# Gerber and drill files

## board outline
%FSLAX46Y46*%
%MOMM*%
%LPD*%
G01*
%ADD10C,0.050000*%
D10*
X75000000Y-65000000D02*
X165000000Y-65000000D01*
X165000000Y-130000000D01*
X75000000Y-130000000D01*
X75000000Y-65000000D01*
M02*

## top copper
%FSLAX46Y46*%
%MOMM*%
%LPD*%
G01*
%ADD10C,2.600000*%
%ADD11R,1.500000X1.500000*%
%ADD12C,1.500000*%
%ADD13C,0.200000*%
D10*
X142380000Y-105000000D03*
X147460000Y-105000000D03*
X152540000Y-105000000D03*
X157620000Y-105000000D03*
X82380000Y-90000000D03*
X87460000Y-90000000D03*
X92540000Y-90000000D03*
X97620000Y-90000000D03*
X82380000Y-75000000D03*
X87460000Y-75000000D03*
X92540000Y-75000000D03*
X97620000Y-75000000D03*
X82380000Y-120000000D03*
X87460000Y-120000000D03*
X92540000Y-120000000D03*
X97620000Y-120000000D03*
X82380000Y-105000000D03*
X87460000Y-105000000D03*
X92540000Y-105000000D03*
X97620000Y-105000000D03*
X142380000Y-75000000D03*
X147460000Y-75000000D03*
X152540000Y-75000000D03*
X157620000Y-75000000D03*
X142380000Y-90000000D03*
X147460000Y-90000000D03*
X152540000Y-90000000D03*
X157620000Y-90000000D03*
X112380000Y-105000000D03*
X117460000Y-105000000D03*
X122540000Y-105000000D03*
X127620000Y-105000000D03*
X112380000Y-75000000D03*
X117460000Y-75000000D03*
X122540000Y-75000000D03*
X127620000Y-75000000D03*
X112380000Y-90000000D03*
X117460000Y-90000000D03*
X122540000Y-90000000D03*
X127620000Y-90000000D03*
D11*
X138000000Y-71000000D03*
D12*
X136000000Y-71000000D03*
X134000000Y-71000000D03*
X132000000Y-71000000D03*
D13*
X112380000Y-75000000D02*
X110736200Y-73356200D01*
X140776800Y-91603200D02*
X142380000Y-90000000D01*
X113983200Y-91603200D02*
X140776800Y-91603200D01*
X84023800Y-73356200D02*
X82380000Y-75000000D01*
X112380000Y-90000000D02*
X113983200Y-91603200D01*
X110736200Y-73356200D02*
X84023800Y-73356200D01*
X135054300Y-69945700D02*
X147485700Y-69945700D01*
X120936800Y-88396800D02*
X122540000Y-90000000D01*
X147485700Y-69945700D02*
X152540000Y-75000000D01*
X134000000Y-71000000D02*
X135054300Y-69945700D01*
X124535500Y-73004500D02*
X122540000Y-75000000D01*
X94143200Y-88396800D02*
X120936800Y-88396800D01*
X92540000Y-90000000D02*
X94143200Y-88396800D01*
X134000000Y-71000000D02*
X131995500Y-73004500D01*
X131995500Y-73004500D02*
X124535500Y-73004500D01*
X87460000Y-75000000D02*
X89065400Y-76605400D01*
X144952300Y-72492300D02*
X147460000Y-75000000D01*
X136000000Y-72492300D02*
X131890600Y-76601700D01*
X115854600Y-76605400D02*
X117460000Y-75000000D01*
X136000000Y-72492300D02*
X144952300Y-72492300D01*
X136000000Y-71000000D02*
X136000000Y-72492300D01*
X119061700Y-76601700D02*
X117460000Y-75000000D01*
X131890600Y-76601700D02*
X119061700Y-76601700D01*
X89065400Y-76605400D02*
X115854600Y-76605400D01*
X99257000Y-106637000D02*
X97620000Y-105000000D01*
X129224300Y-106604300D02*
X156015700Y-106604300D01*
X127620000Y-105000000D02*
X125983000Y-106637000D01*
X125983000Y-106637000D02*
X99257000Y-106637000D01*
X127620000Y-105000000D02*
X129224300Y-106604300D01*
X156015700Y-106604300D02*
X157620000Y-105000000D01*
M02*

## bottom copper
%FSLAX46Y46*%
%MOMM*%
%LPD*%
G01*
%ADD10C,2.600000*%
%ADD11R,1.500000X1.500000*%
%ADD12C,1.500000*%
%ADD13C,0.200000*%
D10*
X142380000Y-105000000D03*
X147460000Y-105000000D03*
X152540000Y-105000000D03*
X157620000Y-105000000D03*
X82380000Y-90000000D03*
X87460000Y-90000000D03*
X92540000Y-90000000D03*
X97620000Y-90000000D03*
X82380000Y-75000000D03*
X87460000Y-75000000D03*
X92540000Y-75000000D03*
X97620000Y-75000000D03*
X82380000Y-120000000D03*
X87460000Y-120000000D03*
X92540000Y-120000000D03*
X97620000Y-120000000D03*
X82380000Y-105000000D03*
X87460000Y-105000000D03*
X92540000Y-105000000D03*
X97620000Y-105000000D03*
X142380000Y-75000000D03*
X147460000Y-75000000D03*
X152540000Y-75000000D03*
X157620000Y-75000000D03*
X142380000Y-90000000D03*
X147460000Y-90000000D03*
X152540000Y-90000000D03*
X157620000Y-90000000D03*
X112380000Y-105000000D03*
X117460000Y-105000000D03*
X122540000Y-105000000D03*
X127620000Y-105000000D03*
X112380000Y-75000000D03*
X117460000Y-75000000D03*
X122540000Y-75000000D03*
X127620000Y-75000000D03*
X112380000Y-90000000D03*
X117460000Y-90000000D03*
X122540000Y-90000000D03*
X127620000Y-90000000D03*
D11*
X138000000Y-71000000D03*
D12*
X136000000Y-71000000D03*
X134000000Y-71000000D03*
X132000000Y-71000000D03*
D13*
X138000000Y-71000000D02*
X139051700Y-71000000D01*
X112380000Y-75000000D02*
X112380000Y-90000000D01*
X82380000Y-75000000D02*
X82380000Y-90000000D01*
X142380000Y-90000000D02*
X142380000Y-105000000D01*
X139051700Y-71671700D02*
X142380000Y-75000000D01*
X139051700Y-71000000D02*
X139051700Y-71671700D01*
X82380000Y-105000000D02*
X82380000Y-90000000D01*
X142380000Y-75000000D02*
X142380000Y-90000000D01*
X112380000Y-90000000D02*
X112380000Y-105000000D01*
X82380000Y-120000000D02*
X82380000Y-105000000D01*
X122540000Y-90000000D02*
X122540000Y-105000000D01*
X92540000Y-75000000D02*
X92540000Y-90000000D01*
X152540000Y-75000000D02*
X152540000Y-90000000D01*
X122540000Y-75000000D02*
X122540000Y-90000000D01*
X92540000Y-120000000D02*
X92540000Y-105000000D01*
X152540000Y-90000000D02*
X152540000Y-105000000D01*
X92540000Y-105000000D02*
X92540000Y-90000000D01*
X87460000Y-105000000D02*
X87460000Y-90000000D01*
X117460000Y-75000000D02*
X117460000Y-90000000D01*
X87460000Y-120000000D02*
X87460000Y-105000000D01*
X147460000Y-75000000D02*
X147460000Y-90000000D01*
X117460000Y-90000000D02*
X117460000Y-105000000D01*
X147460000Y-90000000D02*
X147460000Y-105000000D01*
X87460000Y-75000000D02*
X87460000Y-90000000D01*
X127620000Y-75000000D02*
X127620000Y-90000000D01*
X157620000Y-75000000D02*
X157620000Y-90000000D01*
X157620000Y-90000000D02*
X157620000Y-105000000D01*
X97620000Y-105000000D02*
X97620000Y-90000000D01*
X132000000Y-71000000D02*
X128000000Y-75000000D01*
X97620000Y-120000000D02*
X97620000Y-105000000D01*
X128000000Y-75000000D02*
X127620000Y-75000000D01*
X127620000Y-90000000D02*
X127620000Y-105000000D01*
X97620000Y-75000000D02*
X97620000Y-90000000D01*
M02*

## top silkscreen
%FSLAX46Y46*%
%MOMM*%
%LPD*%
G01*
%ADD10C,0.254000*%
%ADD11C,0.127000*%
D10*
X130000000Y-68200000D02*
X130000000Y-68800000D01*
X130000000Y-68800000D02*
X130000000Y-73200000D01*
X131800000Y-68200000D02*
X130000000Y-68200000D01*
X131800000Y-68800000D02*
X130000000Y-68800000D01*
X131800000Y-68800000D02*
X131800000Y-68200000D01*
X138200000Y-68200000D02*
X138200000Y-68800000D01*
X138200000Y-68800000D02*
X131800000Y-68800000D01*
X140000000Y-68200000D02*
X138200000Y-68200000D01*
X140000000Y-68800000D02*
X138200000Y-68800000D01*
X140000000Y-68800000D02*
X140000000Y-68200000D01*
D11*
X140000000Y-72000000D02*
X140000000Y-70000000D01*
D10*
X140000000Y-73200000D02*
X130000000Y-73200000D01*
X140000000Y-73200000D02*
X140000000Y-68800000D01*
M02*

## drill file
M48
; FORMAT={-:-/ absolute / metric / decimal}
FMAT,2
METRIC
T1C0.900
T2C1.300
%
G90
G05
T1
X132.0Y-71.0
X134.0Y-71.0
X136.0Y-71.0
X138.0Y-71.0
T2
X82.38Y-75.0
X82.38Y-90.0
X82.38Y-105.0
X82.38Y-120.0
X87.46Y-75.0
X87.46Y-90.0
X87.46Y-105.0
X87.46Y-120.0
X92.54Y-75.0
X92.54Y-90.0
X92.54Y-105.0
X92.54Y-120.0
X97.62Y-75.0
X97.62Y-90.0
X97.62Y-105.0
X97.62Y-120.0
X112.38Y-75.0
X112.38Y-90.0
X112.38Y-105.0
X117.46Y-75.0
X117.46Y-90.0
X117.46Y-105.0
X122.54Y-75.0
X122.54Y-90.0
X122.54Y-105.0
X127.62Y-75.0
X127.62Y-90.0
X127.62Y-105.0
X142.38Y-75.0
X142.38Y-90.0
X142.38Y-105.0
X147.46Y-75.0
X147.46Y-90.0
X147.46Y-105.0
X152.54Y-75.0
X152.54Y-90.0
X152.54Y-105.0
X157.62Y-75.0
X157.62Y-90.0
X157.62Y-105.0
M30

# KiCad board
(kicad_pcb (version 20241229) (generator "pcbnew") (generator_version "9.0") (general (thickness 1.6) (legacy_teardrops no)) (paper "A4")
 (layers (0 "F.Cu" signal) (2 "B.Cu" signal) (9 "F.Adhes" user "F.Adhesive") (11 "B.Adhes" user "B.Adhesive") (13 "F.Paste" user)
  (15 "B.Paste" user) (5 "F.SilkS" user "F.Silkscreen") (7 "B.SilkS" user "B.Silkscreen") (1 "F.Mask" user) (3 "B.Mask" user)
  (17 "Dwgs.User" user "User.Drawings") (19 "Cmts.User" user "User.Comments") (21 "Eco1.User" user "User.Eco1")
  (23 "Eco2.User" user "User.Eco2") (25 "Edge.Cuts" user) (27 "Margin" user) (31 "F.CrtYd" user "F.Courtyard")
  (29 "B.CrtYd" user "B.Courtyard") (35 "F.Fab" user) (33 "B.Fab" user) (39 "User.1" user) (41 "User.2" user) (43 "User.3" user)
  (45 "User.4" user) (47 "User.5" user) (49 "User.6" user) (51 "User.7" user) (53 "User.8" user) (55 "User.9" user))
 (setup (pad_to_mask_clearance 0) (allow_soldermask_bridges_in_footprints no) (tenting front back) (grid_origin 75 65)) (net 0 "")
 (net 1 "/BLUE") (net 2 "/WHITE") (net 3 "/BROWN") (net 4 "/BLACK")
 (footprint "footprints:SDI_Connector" (layer "F.Cu") (at 150 105)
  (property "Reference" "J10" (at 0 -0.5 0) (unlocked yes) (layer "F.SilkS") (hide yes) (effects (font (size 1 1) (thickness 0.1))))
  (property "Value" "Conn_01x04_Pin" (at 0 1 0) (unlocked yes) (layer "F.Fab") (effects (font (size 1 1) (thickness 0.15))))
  (pad "1" thru_hole circle (at -7.62 0) (size 2.6 2.6) (drill 1.3) (layers "*.Cu" "*.Mask") (remove_unused_layers no) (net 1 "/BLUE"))
  (pad "2" thru_hole circle (at -2.54 0) (size 2.6 2.6) (drill 1.3) (layers "*.Cu" "*.Mask") (remove_unused_layers no) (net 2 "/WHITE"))
  (pad "3" thru_hole circle (at 2.54 0) (size 2.6 2.6) (drill 1.3) (layers "*.Cu" "*.Mask") (remove_unused_layers no) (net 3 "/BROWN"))
  (pad "4" thru_hole circle (at 7.62 0) (size 2.6 2.6) (drill 1.3) (layers "*.Cu" "*.Mask") (remove_unused_layers no) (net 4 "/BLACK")))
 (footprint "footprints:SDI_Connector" (layer "F.Cu") (at 90 90)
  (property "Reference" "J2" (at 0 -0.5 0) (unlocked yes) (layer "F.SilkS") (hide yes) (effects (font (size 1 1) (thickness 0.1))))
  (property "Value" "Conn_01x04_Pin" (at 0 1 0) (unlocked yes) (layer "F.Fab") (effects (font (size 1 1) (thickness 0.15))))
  (pad "1" thru_hole circle (at -7.62 0) (size 2.6 2.6) (drill 1.3) (layers "*.Cu" "*.Mask") (remove_unused_layers no) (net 1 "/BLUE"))
  (pad "2" thru_hole circle (at -2.54 0) (size 2.6 2.6) (drill 1.3) (layers "*.Cu" "*.Mask") (remove_unused_layers no) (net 2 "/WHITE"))
  (pad "3" thru_hole circle (at 2.54 0) (size 2.6 2.6) (drill 1.3) (layers "*.Cu" "*.Mask") (remove_unused_layers no) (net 3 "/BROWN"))
  (pad "4" thru_hole circle (at 7.62 0) (size 2.6 2.6) (drill 1.3) (layers "*.Cu" "*.Mask") (remove_unused_layers no) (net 4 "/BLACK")))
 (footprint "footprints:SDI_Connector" (layer "F.Cu") (at 90 75)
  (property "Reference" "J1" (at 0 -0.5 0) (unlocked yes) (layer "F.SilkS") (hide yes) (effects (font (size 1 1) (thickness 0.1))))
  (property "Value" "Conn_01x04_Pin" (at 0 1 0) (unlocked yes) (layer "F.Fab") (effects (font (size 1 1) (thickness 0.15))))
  (pad "1" thru_hole circle (at -7.62 0) (size 2.6 2.6) (drill 1.3) (layers "*.Cu" "*.Mask") (remove_unused_layers no) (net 1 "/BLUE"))
  (pad "2" thru_hole circle (at -2.54 0) (size 2.6 2.6) (drill 1.3) (layers "*.Cu" "*.Mask") (remove_unused_layers no) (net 2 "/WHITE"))
  (pad "3" thru_hole circle (at 2.54 0) (size 2.6 2.6) (drill 1.3) (layers "*.Cu" "*.Mask") (remove_unused_layers no) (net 3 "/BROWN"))
  (pad "4" thru_hole circle (at 7.62 0) (size 2.6 2.6) (drill 1.3) (layers "*.Cu" "*.Mask") (remove_unused_layers no) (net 4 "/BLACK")))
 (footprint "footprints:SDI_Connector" (layer "F.Cu") (at 90 120)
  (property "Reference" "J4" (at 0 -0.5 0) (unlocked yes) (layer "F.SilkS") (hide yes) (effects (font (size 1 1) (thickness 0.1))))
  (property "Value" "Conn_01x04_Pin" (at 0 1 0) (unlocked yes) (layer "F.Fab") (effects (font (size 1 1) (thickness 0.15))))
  (pad "1" thru_hole circle (at -7.62 0) (size 2.6 2.6) (drill 1.3) (layers "*.Cu" "*.Mask") (remove_unused_layers no) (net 1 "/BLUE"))
  (pad "2" thru_hole circle (at -2.54 0) (size 2.6 2.6) (drill 1.3) (layers "*.Cu" "*.Mask") (remove_unused_layers no) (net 2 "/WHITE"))
  (pad "3" thru_hole circle (at 2.54 0) (size 2.6 2.6) (drill 1.3) (layers "*.Cu" "*.Mask") (remove_unused_layers no) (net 3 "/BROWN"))
  (pad "4" thru_hole circle (at 7.62 0) (size 2.6 2.6) (drill 1.3) (layers "*.Cu" "*.Mask") (remove_unused_layers no) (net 4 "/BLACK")))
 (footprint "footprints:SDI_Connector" (layer "F.Cu") (at 90 105)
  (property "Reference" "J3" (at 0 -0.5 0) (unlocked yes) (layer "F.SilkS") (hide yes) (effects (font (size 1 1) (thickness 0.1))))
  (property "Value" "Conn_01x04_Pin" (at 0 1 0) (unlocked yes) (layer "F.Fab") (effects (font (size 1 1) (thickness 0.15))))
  (pad "1" thru_hole circle (at -7.62 0) (size 2.6 2.6) (drill 1.3) (layers "*.Cu" "*.Mask") (remove_unused_layers no) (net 1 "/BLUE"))
  (pad "2" thru_hole circle (at -2.54 0) (size 2.6 2.6) (drill 1.3) (layers "*.Cu" "*.Mask") (remove_unused_layers no) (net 2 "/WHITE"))
  (pad "3" thru_hole circle (at 2.54 0) (size 2.6 2.6) (drill 1.3) (layers "*.Cu" "*.Mask") (remove_unused_layers no) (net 3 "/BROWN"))
  (pad "4" thru_hole circle (at 7.62 0) (size 2.6 2.6) (drill 1.3) (layers "*.Cu" "*.Mask") (remove_unused_layers no) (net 4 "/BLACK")))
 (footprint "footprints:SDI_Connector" (layer "F.Cu") (at 150 75)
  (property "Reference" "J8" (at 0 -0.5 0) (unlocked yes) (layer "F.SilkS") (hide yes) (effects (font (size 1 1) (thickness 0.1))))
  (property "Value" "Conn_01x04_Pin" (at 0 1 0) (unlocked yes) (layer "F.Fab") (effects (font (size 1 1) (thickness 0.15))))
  (pad "1" thru_hole circle (at -7.62 0) (size 2.6 2.6) (drill 1.3) (layers "*.Cu" "*.Mask") (remove_unused_layers no) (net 1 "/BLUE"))
  (pad "2" thru_hole circle (at -2.54 0) (size 2.6 2.6) (drill 1.3) (layers "*.Cu" "*.Mask") (remove_unused_layers no) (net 2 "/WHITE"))
  (pad "3" thru_hole circle (at 2.54 0) (size 2.6 2.6) (drill 1.3) (layers "*.Cu" "*.Mask") (remove_unused_layers no) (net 3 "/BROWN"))
  (pad "4" thru_hole circle (at 7.62 0) (size 2.6 2.6) (drill 1.3) (layers "*.Cu" "*.Mask") (remove_unused_layers no) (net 4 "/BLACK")))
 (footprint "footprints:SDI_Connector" (layer "F.Cu") (at 150 90)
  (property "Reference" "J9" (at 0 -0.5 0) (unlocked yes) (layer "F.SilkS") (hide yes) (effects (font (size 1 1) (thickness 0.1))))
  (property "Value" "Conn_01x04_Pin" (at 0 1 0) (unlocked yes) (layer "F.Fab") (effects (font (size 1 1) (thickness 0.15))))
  (pad "1" thru_hole circle (at -7.62 0) (size 2.6 2.6) (drill 1.3) (layers "*.Cu" "*.Mask") (remove_unused_layers no) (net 1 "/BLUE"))
  (pad "2" thru_hole circle (at -2.54 0) (size 2.6 2.6) (drill 1.3) (layers "*.Cu" "*.Mask") (remove_unused_layers no) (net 2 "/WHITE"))
  (pad "3" thru_hole circle (at 2.54 0) (size 2.6 2.6) (drill 1.3) (layers "*.Cu" "*.Mask") (remove_unused_layers no) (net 3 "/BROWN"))
  (pad "4" thru_hole circle (at 7.62 0) (size 2.6 2.6) (drill 1.3) (layers "*.Cu" "*.Mask") (remove_unused_layers no) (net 4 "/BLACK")))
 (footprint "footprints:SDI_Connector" (layer "F.Cu") (at 120 105)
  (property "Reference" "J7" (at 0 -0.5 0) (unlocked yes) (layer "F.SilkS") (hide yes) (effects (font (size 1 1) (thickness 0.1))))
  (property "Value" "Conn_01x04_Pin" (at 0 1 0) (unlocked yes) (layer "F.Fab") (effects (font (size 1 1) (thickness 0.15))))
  (pad "1" thru_hole circle (at -7.62 0) (size 2.6 2.6) (drill 1.3) (layers "*.Cu" "*.Mask") (remove_unused_layers no) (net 1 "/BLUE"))
  (pad "2" thru_hole circle (at -2.54 0) (size 2.6 2.6) (drill 1.3) (layers "*.Cu" "*.Mask") (remove_unused_layers no) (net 2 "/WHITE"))
  (pad "3" thru_hole circle (at 2.54 0) (size 2.6 2.6) (drill 1.3) (layers "*.Cu" "*.Mask") (remove_unused_layers no) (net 3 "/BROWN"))
  (pad "4" thru_hole circle (at 7.62 0) (size 2.6 2.6) (drill 1.3) (layers "*.Cu" "*.Mask") (remove_unused_layers no) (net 4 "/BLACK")))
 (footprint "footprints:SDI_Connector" (layer "F.Cu") (at 120 75)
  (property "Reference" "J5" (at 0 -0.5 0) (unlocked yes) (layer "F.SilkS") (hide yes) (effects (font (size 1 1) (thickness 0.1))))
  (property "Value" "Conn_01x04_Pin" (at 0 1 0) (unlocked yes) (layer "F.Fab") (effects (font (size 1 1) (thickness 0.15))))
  (pad "1" thru_hole circle (at -7.62 0) (size 2.6 2.6) (drill 1.3) (layers "*.Cu" "*.Mask") (remove_unused_layers no) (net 1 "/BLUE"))
  (pad "2" thru_hole circle (at -2.54 0) (size 2.6 2.6) (drill 1.3) (layers "*.Cu" "*.Mask") (remove_unused_layers no) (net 2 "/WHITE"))
  (pad "3" thru_hole circle (at 2.54 0) (size 2.6 2.6) (drill 1.3) (layers "*.Cu" "*.Mask") (remove_unused_layers no) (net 3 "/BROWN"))
  (pad "4" thru_hole circle (at 7.62 0) (size 2.6 2.6) (drill 1.3) (layers "*.Cu" "*.Mask") (remove_unused_layers no) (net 4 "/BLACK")))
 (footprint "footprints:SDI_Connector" (layer "F.Cu") (at 120 90)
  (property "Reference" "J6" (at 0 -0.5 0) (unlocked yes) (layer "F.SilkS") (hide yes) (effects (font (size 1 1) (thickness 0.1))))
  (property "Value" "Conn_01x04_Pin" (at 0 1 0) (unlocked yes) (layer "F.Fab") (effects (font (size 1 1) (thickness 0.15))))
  (pad "1" thru_hole circle (at -7.62 0) (size 2.6 2.6) (drill 1.3) (layers "*.Cu" "*.Mask") (remove_unused_layers no) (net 1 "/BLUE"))
  (pad "2" thru_hole circle (at -2.54 0) (size 2.6 2.6) (drill 1.3) (layers "*.Cu" "*.Mask") (remove_unused_layers no) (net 2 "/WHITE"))
  (pad "3" thru_hole circle (at 2.54 0) (size 2.6 2.6) (drill 1.3) (layers "*.Cu" "*.Mask") (remove_unused_layers no) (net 3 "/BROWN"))
  (pad "4" thru_hole circle (at 7.62 0) (size 2.6 2.6) (drill 1.3) (layers "*.Cu" "*.Mask") (remove_unused_layers no) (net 4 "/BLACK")))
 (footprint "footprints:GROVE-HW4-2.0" (layer "F.Cu") (at 135 71 180)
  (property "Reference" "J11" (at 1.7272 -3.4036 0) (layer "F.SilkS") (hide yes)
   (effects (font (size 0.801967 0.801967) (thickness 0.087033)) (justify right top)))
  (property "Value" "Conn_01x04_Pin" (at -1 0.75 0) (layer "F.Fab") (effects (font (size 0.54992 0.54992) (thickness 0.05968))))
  (fp_line (start 5 2.8) (end 5 2.2) (stroke (width 0.254) (type solid)) (layer "F.SilkS"))
  (fp_line (start 5 2.2) (end 5 -2.2) (stroke (width 0.254) (type solid)) (layer "F.SilkS"))
  (fp_line (start 3.2 2.8) (end 5 2.8) (stroke (width 0.254) (type solid)) (layer "F.SilkS"))
  (fp_line (start 3.2 2.2) (end 5 2.2) (stroke (width 0.254) (type solid)) (layer "F.SilkS"))
  (fp_line (start 3.2 2.2) (end 3.2 2.8) (stroke (width 0.254) (type solid)) (layer "F.SilkS"))
  (fp_line (start -3.2 2.8) (end -3.2 2.2) (stroke (width 0.254) (type solid)) (layer "F.SilkS"))
  (fp_line (start -3.2 2.2) (end 3.2 2.2) (stroke (width 0.254) (type solid)) (layer "F.SilkS"))
  (fp_line (start -5 2.8) (end -3.2 2.8) (stroke (width 0.254) (type solid)) (layer "F.SilkS"))
  (fp_line (start -5 2.2) (end -3.2 2.2) (stroke (width 0.254) (type solid)) (layer "F.SilkS"))
  (fp_line (start -5 2.2) (end -5 2.8) (stroke (width 0.254) (type solid)) (layer "F.SilkS"))
  (fp_line (start -5 -1) (end -5 1) (stroke (width 0.127) (type solid)) (layer "F.SilkS"))
  (fp_line (start -5 -2.2) (end 5 -2.2) (stroke (width 0.254) (type solid)) (layer "F.SilkS"))
  (fp_line (start -5 -2.2) (end -5 2.2) (stroke (width 0.254) (type solid)) (layer "F.SilkS"))
  (pad "1" thru_hole rect (at -3 0 180) (size 1.5 1.5) (drill 0.9) (layers "*.Cu" "*.Mask") (remove_unused_layers no) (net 1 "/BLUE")
   (solder_mask_margin 0.1016) (thermal_bridge_angle 45))
  (pad "2" thru_hole circle (at -1 0 180) (size 1.5 1.5) (drill 0.9) (layers "*.Cu" "*.Mask") (remove_unused_layers no) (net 2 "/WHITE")
   (solder_mask_margin 0.1016))
  (pad "3" thru_hole circle (at 1 0 180) (size 1.5 1.5) (drill 0.9) (layers "*.Cu" "*.Mask") (remove_unused_layers no) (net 3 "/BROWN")
   (solder_mask_margin 0.1016))
  (pad "4" thru_hole circle (at 3 0 180) (size 1.5 1.5) (drill 0.9) (layers "*.Cu" "*.Mask") (remove_unused_layers no) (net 4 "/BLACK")
   (solder_mask_margin 0.1016)))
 (gr_rect (start 75 65) (end 165 130) (stroke (width 0.05) (type solid)) (fill no) (layer "Edge.Cuts"))
 (segment (start 112.38 75) (end 110.7362 73.3562) (width 0.2) (layer "F.Cu") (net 1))
 (segment (start 140.7768 91.6032) (end 142.38 90) (width 0.2) (layer "F.Cu") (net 1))
 (segment (start 113.9832 91.6032) (end 140.7768 91.6032) (width 0.2) (layer "F.Cu") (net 1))
 (segment (start 84.0238 73.3562) (end 82.38 75) (width 0.2) (layer "F.Cu") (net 1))
 (segment (start 112.38 90) (end 113.9832 91.6032) (width 0.2) (layer "F.Cu") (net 1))
 (segment (start 110.7362 73.3562) (end 84.0238 73.3562) (width 0.2) (layer "F.Cu") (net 1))
 (segment (start 138 71) (end 139.0517 71) (width 0.2) (layer "B.Cu") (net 1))
 (segment (start 112.38 75) (end 112.38 90) (width 0.2) (layer "B.Cu") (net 1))
 (segment (start 82.38 75) (end 82.38 90) (width 0.2) (layer "B.Cu") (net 1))
 (segment (start 142.38 90) (end 142.38 105) (width 0.2) (layer "B.Cu") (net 1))
 (segment (start 139.0517 71.6717) (end 142.38 75) (width 0.2) (layer "B.Cu") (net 1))
 (segment (start 139.0517 71) (end 139.0517 71.6717) (width 0.2) (layer "B.Cu") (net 1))
 (segment (start 82.38 105) (end 82.38 90) (width 0.2) (layer "B.Cu") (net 1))
 (segment (start 142.38 75) (end 142.38 90) (width 0.2) (layer "B.Cu") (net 1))
 (segment (start 112.38 90) (end 112.38 105) (width 0.2) (layer "B.Cu") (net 1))
 (segment (start 82.38 120) (end 82.38 105) (width 0.2) (layer "B.Cu") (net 1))
 (segment (start 135.0543 69.9457) (end 147.4857 69.9457) (width 0.2) (layer "F.Cu") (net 3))
 (segment (start 120.9368 88.3968) (end 122.54 90) (width 0.2) (layer "F.Cu") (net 3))
 (segment (start 147.4857 69.9457) (end 152.54 75) (width 0.2) (layer "F.Cu") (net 3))
 (segment (start 134 71) (end 135.0543 69.9457) (width 0.2) (layer "F.Cu") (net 3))
 (segment (start 124.5355 73.0045) (end 122.54 75) (width 0.2) (layer "F.Cu") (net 3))
 (segment (start 94.1432 88.3968) (end 120.9368 88.3968) (width 0.2) (layer "F.Cu") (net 3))
 (segment (start 92.54 90) (end 94.1432 88.3968) (width 0.2) (layer "F.Cu") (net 3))
 (segment (start 134 71) (end 131.9955 73.0045) (width 0.2) (layer "F.Cu") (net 3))
 (segment (start 131.9955 73.0045) (end 124.5355 73.0045) (width 0.2) (layer "F.Cu") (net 3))
 (segment (start 122.54 90) (end 122.54 105) (width 0.2) (layer "B.Cu") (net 3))
 (segment (start 92.54 75) (end 92.54 90) (width 0.2) (layer "B.Cu") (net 3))
 (segment (start 152.54 75) (end 152.54 90) (width 0.2) (layer "B.Cu") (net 3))
 (segment (start 122.54 75) (end 122.54 90) (width 0.2) (layer "B.Cu") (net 3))
 (segment (start 92.54 120) (end 92.54 105) (width 0.2) (layer "B.Cu") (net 3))
 (segment (start 152.54 90) (end 152.54 105) (width 0.2) (layer "B.Cu") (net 3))
 (segment (start 92.54 105) (end 92.54 90) (width 0.2) (layer "B.Cu") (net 3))
 (segment (start 87.46 75) (end 89.0654 76.6054) (width 0.2) (layer "F.Cu") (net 2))
 (segment (start 144.9523 72.4923) (end 147.46 75) (width 0.2) (layer "F.Cu") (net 2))
 (segment (start 136 72.4923) (end 131.8906 76.6017) (width 0.2) (layer "F.Cu") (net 2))
 (segment (start 115.8546 76.6054) (end 117.46 75) (width 0.2) (layer "F.Cu") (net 2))
 (segment (start 136 72.4923) (end 144.9523 72.4923) (width 0.2) (layer "F.Cu") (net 2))
 (segment (start 136 71) (end 136 72.4923) (width 0.2) (layer "F.Cu") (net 2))
 (segment (start 119.0617 76.6017) (end 117.46 75) (width 0.2) (layer "F.Cu") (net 2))
 (segment (start 131.8906 76.6017) (end 119.0617 76.6017) (width 0.2) (layer "F.Cu") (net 2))
 (segment (start 89.0654 76.6054) (end 115.8546 76.6054) (width 0.2) (layer "F.Cu") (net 2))
 (segment (start 87.46 105) (end 87.46 90) (width 0.2) (layer "B.Cu") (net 2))
 (segment (start 117.46 75) (end 117.46 90) (width 0.2) (layer "B.Cu") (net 2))
 (segment (start 87.46 120) (end 87.46 105) (width 0.2) (layer "B.Cu") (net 2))
 (segment (start 147.46 75) (end 147.46 90) (width 0.2) (layer "B.Cu") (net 2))
 (segment (start 117.46 90) (end 117.46 105) (width 0.2) (layer "B.Cu") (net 2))
 (segment (start 147.46 90) (end 147.46 105) (width 0.2) (layer "B.Cu") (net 2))
 (segment (start 87.46 75) (end 87.46 90) (width 0.2) (layer "B.Cu") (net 2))
 (segment (start 99.257 106.637) (end 97.62 105) (width 0.2) (layer "F.Cu") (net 4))
 (segment (start 129.2243 106.6043) (end 156.0157 106.6043) (width 0.2) (layer "F.Cu") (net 4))
 (segment (start 127.62 105) (end 125.983 106.637) (width 0.2) (layer "F.Cu") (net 4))
 (segment (start 125.983 106.637) (end 99.257 106.637) (width 0.2) (layer "F.Cu") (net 4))
 (segment (start 127.62 105) (end 129.2243 106.6043) (width 0.2) (layer "F.Cu") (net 4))
 (segment (start 156.0157 106.6043) (end 157.62 105) (width 0.2) (layer "F.Cu") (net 4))
 (segment (start 127.62 75) (end 127.62 90) (width 0.2) (layer "B.Cu") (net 4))
 (segment (start 157.62 75) (end 157.62 90) (width 0.2) (layer "B.Cu") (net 4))
 (segment (start 157.62 90) (end 157.62 105) (width 0.2) (layer "B.Cu") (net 4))
 (segment (start 97.62 105) (end 97.62 90) (width 0.2) (layer "B.Cu") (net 4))
 (segment (start 132 71) (end 128 75) (width 0.2) (layer "B.Cu") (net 4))
 (segment (start 97.62 120) (end 97.62 105) (width 0.2) (layer "B.Cu") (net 4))
 (segment (start 128 75) (end 127.62 75) (width 0.2) (layer "B.Cu") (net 4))
 (segment (start 127.62 90) (end 127.62 105) (width 0.2) (layer "B.Cu") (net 4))
 (segment (start 97.62 75) (end 97.62 90) (width 0.2) (layer "B.Cu") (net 4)))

